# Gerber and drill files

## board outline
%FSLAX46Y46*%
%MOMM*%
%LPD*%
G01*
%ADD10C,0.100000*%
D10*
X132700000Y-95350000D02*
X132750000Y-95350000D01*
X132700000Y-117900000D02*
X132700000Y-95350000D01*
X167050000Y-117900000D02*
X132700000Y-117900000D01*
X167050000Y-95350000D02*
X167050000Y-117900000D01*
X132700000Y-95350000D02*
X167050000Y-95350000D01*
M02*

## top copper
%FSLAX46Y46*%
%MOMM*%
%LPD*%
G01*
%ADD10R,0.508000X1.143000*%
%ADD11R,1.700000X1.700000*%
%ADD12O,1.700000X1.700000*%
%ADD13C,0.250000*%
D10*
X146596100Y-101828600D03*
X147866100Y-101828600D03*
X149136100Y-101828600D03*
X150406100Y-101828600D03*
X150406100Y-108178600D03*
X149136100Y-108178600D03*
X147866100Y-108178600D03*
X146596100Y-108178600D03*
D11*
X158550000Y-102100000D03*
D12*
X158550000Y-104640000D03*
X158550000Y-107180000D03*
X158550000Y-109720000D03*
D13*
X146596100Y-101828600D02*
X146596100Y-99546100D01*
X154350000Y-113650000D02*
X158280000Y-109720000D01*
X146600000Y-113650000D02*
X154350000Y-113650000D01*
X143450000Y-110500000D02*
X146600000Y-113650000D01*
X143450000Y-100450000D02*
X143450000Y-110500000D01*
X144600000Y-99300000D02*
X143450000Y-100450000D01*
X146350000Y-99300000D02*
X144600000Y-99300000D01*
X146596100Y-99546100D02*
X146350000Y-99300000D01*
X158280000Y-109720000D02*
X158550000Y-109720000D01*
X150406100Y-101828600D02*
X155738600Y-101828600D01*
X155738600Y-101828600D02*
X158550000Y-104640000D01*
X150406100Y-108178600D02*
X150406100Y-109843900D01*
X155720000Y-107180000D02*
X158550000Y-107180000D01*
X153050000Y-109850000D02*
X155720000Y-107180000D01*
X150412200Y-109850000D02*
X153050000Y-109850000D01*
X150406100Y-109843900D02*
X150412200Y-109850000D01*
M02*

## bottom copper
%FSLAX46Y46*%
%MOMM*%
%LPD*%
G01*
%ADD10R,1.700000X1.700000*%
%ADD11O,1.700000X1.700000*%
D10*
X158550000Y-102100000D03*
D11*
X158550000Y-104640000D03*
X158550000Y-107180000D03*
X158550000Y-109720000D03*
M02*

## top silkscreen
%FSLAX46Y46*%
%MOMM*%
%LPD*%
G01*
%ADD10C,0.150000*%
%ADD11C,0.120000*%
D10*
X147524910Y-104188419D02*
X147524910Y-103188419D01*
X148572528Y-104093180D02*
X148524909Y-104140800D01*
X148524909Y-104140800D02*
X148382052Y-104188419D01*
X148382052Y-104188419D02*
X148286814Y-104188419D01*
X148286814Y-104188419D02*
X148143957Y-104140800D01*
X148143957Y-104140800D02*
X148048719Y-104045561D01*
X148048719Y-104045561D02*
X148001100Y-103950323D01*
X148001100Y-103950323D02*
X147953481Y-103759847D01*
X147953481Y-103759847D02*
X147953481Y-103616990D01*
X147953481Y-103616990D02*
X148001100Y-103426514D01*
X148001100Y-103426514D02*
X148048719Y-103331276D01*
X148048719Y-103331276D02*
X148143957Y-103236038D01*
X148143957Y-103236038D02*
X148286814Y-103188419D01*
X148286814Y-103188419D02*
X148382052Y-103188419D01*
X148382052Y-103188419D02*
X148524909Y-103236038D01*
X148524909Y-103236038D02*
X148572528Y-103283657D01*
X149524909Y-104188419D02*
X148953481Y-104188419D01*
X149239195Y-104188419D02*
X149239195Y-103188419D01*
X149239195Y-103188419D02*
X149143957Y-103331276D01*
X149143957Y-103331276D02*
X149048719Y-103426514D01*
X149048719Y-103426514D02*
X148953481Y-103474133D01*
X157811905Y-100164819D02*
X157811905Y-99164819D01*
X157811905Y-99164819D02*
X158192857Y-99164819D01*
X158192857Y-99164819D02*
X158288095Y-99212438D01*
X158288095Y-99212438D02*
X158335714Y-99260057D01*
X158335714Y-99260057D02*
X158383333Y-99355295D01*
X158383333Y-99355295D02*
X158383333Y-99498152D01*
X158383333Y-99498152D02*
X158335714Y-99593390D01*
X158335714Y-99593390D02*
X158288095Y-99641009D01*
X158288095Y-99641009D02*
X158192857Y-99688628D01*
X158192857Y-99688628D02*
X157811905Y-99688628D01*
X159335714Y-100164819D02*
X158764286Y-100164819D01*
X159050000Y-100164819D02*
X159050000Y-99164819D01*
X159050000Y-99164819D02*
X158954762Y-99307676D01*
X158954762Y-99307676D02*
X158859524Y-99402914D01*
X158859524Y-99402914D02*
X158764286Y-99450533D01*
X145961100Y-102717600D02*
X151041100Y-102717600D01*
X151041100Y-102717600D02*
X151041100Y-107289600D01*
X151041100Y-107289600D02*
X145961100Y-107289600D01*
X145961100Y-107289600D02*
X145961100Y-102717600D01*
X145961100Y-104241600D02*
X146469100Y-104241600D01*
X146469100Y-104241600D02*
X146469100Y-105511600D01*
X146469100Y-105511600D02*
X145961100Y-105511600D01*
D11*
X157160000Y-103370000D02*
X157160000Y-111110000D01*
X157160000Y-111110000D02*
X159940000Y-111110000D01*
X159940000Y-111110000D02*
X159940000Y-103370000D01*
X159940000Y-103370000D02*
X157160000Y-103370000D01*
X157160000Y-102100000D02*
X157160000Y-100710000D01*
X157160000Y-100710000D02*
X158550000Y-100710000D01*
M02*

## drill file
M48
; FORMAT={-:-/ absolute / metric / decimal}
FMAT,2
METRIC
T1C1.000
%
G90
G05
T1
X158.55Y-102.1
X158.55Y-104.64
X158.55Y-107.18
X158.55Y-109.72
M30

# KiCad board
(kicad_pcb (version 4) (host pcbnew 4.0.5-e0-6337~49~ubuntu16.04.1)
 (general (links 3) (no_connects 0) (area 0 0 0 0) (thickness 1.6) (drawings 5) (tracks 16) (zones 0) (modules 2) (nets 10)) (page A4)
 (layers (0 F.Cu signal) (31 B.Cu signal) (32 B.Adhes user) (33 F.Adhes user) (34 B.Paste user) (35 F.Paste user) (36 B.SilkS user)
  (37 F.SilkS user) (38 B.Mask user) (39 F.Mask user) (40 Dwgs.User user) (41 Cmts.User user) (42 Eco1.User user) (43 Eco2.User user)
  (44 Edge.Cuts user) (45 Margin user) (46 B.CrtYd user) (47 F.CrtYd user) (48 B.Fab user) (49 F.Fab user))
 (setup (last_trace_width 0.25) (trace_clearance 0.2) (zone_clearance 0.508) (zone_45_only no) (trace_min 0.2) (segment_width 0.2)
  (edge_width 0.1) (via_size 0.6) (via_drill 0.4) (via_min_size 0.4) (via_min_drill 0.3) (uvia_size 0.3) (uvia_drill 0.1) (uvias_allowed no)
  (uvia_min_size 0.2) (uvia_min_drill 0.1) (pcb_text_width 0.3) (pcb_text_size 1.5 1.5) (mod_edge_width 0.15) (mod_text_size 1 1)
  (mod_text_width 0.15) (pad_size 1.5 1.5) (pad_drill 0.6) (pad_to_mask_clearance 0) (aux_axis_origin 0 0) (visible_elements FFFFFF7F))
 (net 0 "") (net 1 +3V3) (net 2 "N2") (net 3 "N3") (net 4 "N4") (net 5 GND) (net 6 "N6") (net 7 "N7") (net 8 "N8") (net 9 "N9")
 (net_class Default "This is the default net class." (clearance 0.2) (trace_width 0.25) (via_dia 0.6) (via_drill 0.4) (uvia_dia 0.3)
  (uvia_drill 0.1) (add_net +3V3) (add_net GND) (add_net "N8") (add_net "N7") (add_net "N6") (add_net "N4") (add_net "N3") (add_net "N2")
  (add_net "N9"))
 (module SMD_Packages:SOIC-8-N (layer F.Cu) (at 148.5011 105.0036)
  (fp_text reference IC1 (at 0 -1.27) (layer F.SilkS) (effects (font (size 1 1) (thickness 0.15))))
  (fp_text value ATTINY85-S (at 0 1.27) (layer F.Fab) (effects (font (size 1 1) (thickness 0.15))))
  (fp_line (start -2.54 -2.286) (end 2.54 -2.286) (layer F.SilkS) (width 0.15))
  (fp_line (start 2.54 -2.286) (end 2.54 2.286) (layer F.SilkS) (width 0.15))
  (fp_line (start 2.54 2.286) (end -2.54 2.286) (layer F.SilkS) (width 0.15))
  (fp_line (start -2.54 2.286) (end -2.54 -2.286) (layer F.SilkS) (width 0.15))
  (fp_line (start -2.54 -0.762) (end -2.032 -0.762) (layer F.SilkS) (width 0.15))
  (fp_line (start -2.032 -0.762) (end -2.032 0.508) (layer F.SilkS) (width 0.15))
  (fp_line (start -2.032 0.508) (end -2.54 0.508) (layer F.SilkS) (width 0.15))
  (pad 8 smd rect (at -1.905 -3.175) (size 0.508 1.143) (layers F.Cu F.Paste F.Mask) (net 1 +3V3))
  (pad 7 smd rect (at -0.635 -3.175) (size 0.508 1.143) (layers F.Cu F.Paste F.Mask) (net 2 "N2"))
  (pad 6 smd rect (at 0.635 -3.175) (size 0.508 1.143) (layers F.Cu F.Paste F.Mask) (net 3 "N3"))
  (pad 5 smd rect (at 1.905 -3.175) (size 0.508 1.143) (layers F.Cu F.Paste F.Mask) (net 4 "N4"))
  (pad 4 smd rect (at 1.905 3.175) (size 0.508 1.143) (layers F.Cu F.Paste F.Mask) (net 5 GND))
  (pad 3 smd rect (at 0.635 3.175) (size 0.508 1.143) (layers F.Cu F.Paste F.Mask) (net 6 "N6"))
  (pad 2 smd rect (at -0.635 3.175) (size 0.508 1.143) (layers F.Cu F.Paste F.Mask) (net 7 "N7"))
  (pad 1 smd rect (at -1.905 3.175) (size 0.508 1.143) (layers F.Cu F.Paste F.Mask) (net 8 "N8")))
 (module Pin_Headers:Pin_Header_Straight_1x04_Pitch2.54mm (layer F.Cu) (at 158.55 102.1)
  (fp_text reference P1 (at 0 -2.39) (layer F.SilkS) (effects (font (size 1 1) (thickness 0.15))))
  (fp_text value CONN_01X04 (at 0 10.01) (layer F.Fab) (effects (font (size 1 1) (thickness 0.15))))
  (fp_line (start -1.39 1.27) (end -1.39 9.01) (layer F.SilkS) (width 0.12))
  (fp_line (start -1.39 9.01) (end 1.39 9.01) (layer F.SilkS) (width 0.12))
  (fp_line (start 1.39 9.01) (end 1.39 1.27) (layer F.SilkS) (width 0.12))
  (fp_line (start 1.39 1.27) (end -1.39 1.27) (layer F.SilkS) (width 0.12))
  (fp_line (start -1.39 0) (end -1.39 -1.39) (layer F.SilkS) (width 0.12))
  (fp_line (start -1.39 -1.39) (end 0 -1.39) (layer F.SilkS) (width 0.12))
  (pad 1 thru_hole rect (at 0 0) (size 1.7 1.7) (drill 1) (layers *.Cu *.Mask) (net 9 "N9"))
  (pad 2 thru_hole oval (at 0 2.54) (size 1.7 1.7) (drill 1) (layers *.Cu *.Mask) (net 4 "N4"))
  (pad 3 thru_hole oval (at 0 5.08) (size 1.7 1.7) (drill 1) (layers *.Cu *.Mask) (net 5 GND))
  (pad 4 thru_hole oval (at 0 7.62) (size 1.7 1.7) (drill 1) (layers *.Cu *.Mask) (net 1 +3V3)))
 (gr_line (start 132.7 95.35) (end 132.75 95.35) (angle 90) (layer Edge.Cuts) (width 0.1))
 (gr_line (start 132.7 117.9) (end 132.7 95.35) (angle 90) (layer Edge.Cuts) (width 0.1))
 (gr_line (start 167.05 117.9) (end 132.7 117.9) (angle 90) (layer Edge.Cuts) (width 0.1))
 (gr_line (start 167.05 95.35) (end 167.05 117.9) (angle 90) (layer Edge.Cuts) (width 0.1))
 (gr_line (start 132.7 95.35) (end 167.05 95.35) (angle 90) (layer Edge.Cuts) (width 0.1))
 (segment (start 146.5961 101.8286) (end 146.5961 99.5461) (width 0.25) (layer F.Cu) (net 1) (status 400000))
 (segment (start 154.35 113.65) (end 158.28 109.72) (width 0.25) (layer F.Cu) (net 1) (status 800000))
 (segment (start 146.6 113.65) (end 154.35 113.65) (width 0.25) (layer F.Cu) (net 1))
 (segment (start 143.45 110.5) (end 146.6 113.65) (width 0.25) (layer F.Cu) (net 1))
 (segment (start 143.45 100.45) (end 143.45 110.5) (width 0.25) (layer F.Cu) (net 1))
 (segment (start 144.6 99.3) (end 143.45 100.45) (width 0.25) (layer F.Cu) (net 1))
 (segment (start 146.35 99.3) (end 144.6 99.3) (width 0.25) (layer F.Cu) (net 1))
 (segment (start 146.5961 99.5461) (end 146.35 99.3) (width 0.25) (layer F.Cu) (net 1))
 (segment (start 158.28 109.72) (end 158.55 109.72) (width 0.25) (layer F.Cu) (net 1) (status C00000))
 (segment (start 150.4061 101.8286) (end 155.7386 101.8286) (width 0.25) (layer F.Cu) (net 4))
 (segment (start 155.7386 101.8286) (end 158.55 104.64) (width 0.25) (layer F.Cu) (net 4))
 (segment (start 150.4061 108.1786) (end 150.4061 109.8439) (width 0.25) (layer F.Cu) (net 5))
 (segment (start 155.72 107.18) (end 158.55 107.18) (width 0.25) (layer F.Cu) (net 5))
 (segment (start 153.05 109.85) (end 155.72 107.18) (width 0.25) (layer F.Cu) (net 5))
 (segment (start 150.4122 109.85) (end 153.05 109.85) (width 0.25) (layer F.Cu) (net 5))
 (segment (start 150.4061 109.8439) (end 150.4122 109.85) (width 0.25) (layer F.Cu) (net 5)))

